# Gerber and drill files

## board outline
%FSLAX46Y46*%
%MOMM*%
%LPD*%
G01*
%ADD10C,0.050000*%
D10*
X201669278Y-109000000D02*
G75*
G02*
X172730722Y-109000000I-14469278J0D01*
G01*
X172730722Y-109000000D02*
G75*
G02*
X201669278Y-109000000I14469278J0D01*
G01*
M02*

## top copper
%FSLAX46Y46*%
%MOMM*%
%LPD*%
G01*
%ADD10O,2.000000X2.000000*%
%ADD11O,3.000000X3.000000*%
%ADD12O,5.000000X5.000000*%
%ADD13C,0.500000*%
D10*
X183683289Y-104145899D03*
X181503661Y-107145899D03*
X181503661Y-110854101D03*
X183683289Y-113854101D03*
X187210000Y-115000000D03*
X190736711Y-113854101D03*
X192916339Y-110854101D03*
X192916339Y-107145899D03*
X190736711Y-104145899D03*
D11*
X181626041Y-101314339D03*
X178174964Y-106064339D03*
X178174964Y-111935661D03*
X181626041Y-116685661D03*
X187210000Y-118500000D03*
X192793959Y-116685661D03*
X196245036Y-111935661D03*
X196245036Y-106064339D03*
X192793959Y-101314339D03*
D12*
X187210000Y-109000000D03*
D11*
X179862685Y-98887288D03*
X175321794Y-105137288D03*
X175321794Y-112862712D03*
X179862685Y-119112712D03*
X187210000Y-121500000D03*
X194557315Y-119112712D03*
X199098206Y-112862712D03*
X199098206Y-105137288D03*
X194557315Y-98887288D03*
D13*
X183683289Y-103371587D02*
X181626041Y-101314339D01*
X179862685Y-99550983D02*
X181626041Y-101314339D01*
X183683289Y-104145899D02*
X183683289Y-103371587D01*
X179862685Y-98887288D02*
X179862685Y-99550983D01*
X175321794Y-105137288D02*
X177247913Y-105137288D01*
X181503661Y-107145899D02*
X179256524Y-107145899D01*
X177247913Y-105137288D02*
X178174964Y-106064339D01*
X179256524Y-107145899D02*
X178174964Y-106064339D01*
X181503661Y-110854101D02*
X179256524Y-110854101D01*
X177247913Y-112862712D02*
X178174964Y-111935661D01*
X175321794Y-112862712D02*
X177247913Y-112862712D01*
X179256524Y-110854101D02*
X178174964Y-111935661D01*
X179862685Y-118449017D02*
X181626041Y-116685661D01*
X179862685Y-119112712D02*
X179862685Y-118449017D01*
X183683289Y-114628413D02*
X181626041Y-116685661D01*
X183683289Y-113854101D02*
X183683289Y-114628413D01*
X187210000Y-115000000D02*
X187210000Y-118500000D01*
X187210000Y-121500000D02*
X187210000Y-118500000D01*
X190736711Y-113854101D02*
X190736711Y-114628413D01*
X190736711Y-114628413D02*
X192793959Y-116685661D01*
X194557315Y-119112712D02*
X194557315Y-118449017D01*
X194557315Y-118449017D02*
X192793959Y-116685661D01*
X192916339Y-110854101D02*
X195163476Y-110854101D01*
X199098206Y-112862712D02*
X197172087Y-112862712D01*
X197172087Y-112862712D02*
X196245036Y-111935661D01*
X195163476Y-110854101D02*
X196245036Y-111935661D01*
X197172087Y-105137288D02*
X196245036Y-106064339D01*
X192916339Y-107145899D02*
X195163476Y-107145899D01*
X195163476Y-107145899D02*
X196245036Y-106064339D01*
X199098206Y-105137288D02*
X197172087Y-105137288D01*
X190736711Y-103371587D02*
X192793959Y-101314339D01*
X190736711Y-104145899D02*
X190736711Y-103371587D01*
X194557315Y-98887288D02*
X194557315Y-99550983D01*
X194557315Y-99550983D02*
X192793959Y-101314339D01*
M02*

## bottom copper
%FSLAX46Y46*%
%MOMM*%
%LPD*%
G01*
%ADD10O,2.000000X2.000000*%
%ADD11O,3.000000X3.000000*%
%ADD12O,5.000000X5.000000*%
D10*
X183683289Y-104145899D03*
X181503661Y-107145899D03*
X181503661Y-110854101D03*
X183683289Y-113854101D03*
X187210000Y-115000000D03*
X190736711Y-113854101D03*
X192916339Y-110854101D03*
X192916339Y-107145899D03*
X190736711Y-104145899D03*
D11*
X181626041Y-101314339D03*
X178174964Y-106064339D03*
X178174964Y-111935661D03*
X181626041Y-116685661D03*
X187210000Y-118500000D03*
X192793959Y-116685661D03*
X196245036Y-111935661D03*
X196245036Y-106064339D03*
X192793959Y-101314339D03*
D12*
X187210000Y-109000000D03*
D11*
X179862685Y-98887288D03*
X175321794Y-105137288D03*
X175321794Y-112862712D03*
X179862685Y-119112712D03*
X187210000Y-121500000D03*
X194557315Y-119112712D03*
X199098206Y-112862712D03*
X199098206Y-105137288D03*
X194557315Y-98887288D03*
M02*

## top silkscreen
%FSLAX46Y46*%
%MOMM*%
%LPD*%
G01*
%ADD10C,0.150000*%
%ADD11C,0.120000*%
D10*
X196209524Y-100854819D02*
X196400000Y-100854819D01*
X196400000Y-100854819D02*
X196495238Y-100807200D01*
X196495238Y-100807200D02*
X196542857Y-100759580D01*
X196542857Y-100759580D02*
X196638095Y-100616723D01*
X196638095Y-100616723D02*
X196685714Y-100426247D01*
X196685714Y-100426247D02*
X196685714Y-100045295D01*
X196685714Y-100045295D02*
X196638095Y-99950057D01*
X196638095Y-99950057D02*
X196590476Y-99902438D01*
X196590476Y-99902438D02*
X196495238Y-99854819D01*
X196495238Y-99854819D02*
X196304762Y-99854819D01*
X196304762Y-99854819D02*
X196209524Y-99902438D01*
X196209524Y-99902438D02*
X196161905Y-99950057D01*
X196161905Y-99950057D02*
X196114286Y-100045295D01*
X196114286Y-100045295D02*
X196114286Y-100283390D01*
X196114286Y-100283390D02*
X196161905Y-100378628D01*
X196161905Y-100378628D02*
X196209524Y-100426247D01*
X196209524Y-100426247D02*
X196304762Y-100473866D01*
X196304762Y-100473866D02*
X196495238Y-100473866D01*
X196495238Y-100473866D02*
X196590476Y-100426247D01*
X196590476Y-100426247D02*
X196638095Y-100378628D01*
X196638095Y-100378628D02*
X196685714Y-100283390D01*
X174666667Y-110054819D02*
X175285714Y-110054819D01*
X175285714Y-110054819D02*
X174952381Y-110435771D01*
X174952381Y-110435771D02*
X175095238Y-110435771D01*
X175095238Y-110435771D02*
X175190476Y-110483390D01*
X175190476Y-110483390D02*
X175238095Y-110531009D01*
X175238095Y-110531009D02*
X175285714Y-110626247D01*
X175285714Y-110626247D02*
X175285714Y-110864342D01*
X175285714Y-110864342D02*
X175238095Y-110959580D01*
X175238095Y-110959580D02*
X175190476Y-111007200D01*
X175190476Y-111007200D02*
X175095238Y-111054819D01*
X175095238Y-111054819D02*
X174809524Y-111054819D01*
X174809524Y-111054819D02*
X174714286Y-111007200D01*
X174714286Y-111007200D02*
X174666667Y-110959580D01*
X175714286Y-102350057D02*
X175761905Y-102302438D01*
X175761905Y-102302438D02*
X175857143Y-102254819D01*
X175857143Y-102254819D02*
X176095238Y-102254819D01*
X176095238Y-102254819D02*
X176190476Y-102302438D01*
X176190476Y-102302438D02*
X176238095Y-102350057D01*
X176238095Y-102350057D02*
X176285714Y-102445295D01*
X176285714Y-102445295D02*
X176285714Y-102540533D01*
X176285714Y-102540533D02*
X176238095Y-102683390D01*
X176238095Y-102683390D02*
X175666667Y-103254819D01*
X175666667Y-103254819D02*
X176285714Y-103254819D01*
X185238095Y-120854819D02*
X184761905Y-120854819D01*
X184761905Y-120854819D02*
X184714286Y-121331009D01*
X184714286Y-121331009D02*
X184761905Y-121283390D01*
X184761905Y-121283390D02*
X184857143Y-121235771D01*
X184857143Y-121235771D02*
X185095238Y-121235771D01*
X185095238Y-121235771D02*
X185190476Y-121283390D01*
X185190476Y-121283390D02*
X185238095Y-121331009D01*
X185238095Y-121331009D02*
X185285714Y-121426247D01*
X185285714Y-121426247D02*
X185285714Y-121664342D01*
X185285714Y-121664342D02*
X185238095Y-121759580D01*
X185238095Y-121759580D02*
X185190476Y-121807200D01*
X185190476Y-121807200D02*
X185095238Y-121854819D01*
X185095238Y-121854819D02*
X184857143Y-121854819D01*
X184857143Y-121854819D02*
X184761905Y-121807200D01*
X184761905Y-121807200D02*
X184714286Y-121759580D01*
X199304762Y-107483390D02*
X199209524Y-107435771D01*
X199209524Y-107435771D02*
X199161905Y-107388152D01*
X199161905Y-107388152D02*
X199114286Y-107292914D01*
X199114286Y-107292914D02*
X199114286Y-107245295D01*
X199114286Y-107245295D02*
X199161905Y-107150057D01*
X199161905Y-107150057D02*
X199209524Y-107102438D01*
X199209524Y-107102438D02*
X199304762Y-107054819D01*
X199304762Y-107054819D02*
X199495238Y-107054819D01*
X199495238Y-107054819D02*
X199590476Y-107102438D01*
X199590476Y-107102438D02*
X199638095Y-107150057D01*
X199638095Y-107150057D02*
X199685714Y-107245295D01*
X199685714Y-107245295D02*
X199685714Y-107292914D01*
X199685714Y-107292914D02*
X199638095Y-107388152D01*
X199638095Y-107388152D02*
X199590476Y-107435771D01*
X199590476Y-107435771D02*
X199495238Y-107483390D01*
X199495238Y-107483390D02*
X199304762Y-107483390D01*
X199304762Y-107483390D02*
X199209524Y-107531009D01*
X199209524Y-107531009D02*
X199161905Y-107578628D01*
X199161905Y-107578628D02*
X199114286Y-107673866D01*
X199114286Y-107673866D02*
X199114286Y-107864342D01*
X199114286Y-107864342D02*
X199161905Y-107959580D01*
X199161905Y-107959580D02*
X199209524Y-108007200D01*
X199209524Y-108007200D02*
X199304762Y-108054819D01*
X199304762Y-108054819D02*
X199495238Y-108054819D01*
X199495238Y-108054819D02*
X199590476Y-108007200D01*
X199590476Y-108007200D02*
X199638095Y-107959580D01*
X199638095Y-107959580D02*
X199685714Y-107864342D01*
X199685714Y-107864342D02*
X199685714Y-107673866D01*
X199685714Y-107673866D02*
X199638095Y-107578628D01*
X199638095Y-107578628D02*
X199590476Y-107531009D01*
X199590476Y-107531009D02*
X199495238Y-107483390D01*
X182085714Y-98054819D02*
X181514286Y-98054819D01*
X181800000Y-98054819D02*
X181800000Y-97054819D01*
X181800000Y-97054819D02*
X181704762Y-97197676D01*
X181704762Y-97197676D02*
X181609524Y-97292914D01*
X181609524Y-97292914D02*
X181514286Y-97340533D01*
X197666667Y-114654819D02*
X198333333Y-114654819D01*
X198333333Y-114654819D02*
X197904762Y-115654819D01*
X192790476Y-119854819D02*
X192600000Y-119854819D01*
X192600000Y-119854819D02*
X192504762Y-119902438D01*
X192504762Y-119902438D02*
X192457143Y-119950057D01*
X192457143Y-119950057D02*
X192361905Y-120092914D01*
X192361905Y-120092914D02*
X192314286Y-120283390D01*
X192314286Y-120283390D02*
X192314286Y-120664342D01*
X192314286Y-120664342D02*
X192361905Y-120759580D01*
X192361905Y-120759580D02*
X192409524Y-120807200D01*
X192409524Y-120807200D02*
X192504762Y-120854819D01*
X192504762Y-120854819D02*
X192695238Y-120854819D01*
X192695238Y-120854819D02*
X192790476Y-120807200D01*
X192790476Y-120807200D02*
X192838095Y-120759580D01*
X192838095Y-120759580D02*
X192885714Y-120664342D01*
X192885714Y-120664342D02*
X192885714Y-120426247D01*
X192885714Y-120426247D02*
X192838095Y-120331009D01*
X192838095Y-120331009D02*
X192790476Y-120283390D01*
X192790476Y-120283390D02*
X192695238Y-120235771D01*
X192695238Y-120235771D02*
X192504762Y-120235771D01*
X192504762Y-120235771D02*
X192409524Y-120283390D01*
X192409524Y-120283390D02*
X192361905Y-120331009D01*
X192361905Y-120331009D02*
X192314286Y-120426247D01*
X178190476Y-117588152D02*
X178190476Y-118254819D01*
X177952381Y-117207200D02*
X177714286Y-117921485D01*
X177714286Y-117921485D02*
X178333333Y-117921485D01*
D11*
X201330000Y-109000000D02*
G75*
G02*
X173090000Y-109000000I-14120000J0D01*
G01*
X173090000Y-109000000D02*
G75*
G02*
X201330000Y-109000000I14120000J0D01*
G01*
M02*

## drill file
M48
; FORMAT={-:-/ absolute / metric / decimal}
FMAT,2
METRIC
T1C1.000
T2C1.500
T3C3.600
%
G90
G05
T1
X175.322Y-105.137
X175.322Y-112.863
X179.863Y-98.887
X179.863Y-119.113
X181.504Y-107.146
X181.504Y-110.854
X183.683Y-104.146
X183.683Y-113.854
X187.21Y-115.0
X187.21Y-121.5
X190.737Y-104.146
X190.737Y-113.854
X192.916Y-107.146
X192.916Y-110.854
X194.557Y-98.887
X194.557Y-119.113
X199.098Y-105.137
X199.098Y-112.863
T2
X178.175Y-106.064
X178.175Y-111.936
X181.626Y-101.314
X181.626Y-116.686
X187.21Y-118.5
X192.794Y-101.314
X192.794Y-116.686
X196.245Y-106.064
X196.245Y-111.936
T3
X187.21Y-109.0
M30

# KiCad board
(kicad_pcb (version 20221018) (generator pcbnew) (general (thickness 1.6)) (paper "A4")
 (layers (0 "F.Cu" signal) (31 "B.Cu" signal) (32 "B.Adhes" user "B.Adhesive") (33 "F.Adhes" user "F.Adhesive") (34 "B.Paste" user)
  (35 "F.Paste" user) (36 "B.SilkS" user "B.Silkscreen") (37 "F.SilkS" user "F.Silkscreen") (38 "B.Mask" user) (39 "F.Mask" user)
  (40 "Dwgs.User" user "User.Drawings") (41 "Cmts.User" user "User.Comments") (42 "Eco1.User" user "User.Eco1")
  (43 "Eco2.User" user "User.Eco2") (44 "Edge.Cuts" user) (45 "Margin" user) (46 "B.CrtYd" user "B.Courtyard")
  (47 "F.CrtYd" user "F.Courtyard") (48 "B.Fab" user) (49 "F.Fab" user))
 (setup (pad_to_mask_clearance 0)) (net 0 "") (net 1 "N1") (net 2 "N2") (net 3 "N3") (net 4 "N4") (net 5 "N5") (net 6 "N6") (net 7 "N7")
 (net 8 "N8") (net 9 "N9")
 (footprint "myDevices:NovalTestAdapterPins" (layer "F.Cu") (at 187.21 109)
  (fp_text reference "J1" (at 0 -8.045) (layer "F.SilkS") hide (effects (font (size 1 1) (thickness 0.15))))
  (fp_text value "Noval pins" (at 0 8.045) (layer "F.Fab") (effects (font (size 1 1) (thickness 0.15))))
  (pad "1" thru_hole oval (at -3.526711 -4.854101) (size 2 2) (drill 1) (layers "*.Cu" "*.Mask") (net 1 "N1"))
  (pad "2" thru_hole oval (at -5.706339 -1.854101) (size 2 2) (drill 1) (layers "*.Cu" "*.Mask") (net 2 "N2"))
  (pad "3" thru_hole oval (at -5.706339 1.854101) (size 2 2) (drill 1) (layers "*.Cu" "*.Mask") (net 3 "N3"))
  (pad "4" thru_hole oval (at -3.526711 4.854101) (size 2 2) (drill 1) (layers "*.Cu" "*.Mask") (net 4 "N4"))
  (pad "5" thru_hole oval (at 0 6) (size 2 2) (drill 1) (layers "*.Cu" "*.Mask") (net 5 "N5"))
  (pad "6" thru_hole oval (at 3.526711 4.854101) (size 2 2) (drill 1) (layers "*.Cu" "*.Mask") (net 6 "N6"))
  (pad "7" thru_hole oval (at 5.706339 1.854101) (size 2 2) (drill 1) (layers "*.Cu" "*.Mask") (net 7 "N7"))
  (pad "8" thru_hole oval (at 5.706339 -1.854101) (size 2 2) (drill 1) (layers "*.Cu" "*.Mask") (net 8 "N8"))
  (pad "9" thru_hole oval (at 3.526711 -4.854101) (size 2 2) (drill 1) (layers "*.Cu" "*.Mask") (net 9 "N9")))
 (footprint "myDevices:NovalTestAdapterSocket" (layer "F.Cu") (at 187.21 109)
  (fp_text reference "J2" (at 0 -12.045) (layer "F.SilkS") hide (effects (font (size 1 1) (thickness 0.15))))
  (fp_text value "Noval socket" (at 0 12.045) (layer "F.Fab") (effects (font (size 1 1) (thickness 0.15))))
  (pad "1" thru_hole oval (at -5.583959 -7.685661) (size 3 3) (drill 1.5) (layers "*.Cu" "*.Mask") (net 1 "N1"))
  (pad "2" thru_hole oval (at -9.035036 -2.935661) (size 3 3) (drill 1.5) (layers "*.Cu" "*.Mask") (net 2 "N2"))
  (pad "3" thru_hole oval (at -9.035036 2.935661) (size 3 3) (drill 1.5) (layers "*.Cu" "*.Mask") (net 3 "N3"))
  (pad "4" thru_hole oval (at -5.583959 7.685661) (size 3 3) (drill 1.5) (layers "*.Cu" "*.Mask") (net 4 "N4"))
  (pad "5" thru_hole oval (at 0 9.5) (size 3 3) (drill 1.5) (layers "*.Cu" "*.Mask") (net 5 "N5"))
  (pad "6" thru_hole oval (at 5.583959 7.685661) (size 3 3) (drill 1.5) (layers "*.Cu" "*.Mask") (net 6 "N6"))
  (pad "7" thru_hole oval (at 9.035036 2.935661) (size 3 3) (drill 1.5) (layers "*.Cu" "*.Mask") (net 7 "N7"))
  (pad "8" thru_hole oval (at 9.035036 -2.935661) (size 3 3) (drill 1.5) (layers "*.Cu" "*.Mask") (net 8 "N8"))
  (pad "9" thru_hole oval (at 5.583959 -7.685661) (size 3 3) (drill 1.5) (layers "*.Cu" "*.Mask") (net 9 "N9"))
  (pad "10" thru_hole oval (at 0 0) (size 5 5) (drill 3.6) (layers "*.Cu" "*.Mask")))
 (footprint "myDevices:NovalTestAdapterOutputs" (layer "F.Cu") (at 187.21 109)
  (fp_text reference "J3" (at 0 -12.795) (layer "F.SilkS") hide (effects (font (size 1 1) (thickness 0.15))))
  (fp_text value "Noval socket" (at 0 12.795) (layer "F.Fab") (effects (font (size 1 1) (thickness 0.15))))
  (fp_circle (center 0 0) (end 0 14.12) (stroke (width 0.12) (type solid)) (fill none) (layer "F.SilkS"))
  (pad "1" thru_hole oval (at -7.347315 -10.112712) (size 3 3) (drill 1) (layers "*.Cu" "*.Mask") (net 1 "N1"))
  (pad "2" thru_hole oval (at -11.888206 -3.862712) (size 3 3) (drill 1) (layers "*.Cu" "*.Mask") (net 2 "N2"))
  (pad "3" thru_hole oval (at -11.888206 3.862712) (size 3 3) (drill 1) (layers "*.Cu" "*.Mask") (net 3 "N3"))
  (pad "4" thru_hole oval (at -7.347315 10.112712) (size 3 3) (drill 1) (layers "*.Cu" "*.Mask") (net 4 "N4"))
  (pad "5" thru_hole oval (at 0 12.5) (size 3 3) (drill 1) (layers "*.Cu" "*.Mask") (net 5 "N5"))
  (pad "6" thru_hole oval (at 7.347315 10.112712) (size 3 3) (drill 1) (layers "*.Cu" "*.Mask") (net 6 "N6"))
  (pad "7" thru_hole oval (at 11.888206 3.862712) (size 3 3) (drill 1) (layers "*.Cu" "*.Mask") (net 7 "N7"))
  (pad "8" thru_hole oval (at 11.888206 -3.862712) (size 3 3) (drill 1) (layers "*.Cu" "*.Mask") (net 8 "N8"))
  (pad "9" thru_hole oval (at 7.347315 -10.112712) (size 3 3) (drill 1) (layers "*.Cu" "*.Mask") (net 9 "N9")))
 (gr_circle (center 187.2 109) (end 198.2 118.4) (stroke (width 0.05) (type solid)) (fill none) (layer "Edge.Cuts"))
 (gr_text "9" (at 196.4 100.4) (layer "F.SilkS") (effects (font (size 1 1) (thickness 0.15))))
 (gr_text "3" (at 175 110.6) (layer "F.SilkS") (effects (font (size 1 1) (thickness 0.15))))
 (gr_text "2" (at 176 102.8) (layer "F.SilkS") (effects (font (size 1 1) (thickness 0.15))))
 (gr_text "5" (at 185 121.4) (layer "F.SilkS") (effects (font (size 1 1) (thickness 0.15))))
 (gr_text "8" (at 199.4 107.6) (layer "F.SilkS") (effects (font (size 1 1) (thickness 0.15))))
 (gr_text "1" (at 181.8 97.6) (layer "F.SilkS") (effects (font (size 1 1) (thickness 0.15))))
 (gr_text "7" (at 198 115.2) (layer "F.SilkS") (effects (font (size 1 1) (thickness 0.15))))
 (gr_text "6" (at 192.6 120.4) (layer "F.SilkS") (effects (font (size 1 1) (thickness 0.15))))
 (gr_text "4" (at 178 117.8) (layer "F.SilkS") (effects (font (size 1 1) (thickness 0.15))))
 (segment (start 183.683289 103.371587) (end 181.626041 101.314339) (width 0.5) (layer "F.Cu") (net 1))
 (segment (start 179.862685 99.550983) (end 181.626041 101.314339) (width 0.5) (layer "F.Cu") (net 1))
 (segment (start 183.683289 104.145899) (end 183.683289 103.371587) (width 0.5) (layer "F.Cu") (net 1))
 (segment (start 179.862685 98.887288) (end 179.862685 99.550983) (width 0.5) (layer "F.Cu") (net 1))
 (segment (start 175.321794 105.137288) (end 177.247913 105.137288) (width 0.5) (layer "F.Cu") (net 2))
 (segment (start 181.503661 107.145899) (end 179.256524 107.145899) (width 0.5) (layer "F.Cu") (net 2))
 (segment (start 177.247913 105.137288) (end 178.174964 106.064339) (width 0.5) (layer "F.Cu") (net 2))
 (segment (start 179.256524 107.145899) (end 178.174964 106.064339) (width 0.5) (layer "F.Cu") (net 2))
 (segment (start 181.503661 110.854101) (end 179.256524 110.854101) (width 0.5) (layer "F.Cu") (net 3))
 (segment (start 177.247913 112.862712) (end 178.174964 111.935661) (width 0.5) (layer "F.Cu") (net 3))
 (segment (start 175.321794 112.862712) (end 177.247913 112.862712) (width 0.5) (layer "F.Cu") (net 3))
 (segment (start 179.256524 110.854101) (end 178.174964 111.935661) (width 0.5) (layer "F.Cu") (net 3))
 (segment (start 179.862685 118.449017) (end 181.626041 116.685661) (width 0.5) (layer "F.Cu") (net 4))
 (segment (start 179.862685 119.112712) (end 179.862685 118.449017) (width 0.5) (layer "F.Cu") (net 4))
 (segment (start 183.683289 114.628413) (end 181.626041 116.685661) (width 0.5) (layer "F.Cu") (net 4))
 (segment (start 183.683289 113.854101) (end 183.683289 114.628413) (width 0.5) (layer "F.Cu") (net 4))
 (segment (start 187.21 115) (end 187.21 118.5) (width 0.5) (layer "F.Cu") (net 5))
 (segment (start 187.21 121.5) (end 187.21 118.5) (width 0.5) (layer "F.Cu") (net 5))
 (segment (start 190.736711 113.854101) (end 190.736711 114.628413) (width 0.5) (layer "F.Cu") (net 6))
 (segment (start 190.736711 114.628413) (end 192.793959 116.685661) (width 0.5) (layer "F.Cu") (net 6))
 (segment (start 194.557315 119.112712) (end 194.557315 118.449017) (width 0.5) (layer "F.Cu") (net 6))
 (segment (start 194.557315 118.449017) (end 192.793959 116.685661) (width 0.5) (layer "F.Cu") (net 6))
 (segment (start 192.916339 110.854101) (end 195.163476 110.854101) (width 0.5) (layer "F.Cu") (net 7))
 (segment (start 199.098206 112.862712) (end 197.172087 112.862712) (width 0.5) (layer "F.Cu") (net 7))
 (segment (start 197.172087 112.862712) (end 196.245036 111.935661) (width 0.5) (layer "F.Cu") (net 7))
 (segment (start 195.163476 110.854101) (end 196.245036 111.935661) (width 0.5) (layer "F.Cu") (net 7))
 (segment (start 197.172087 105.137288) (end 196.245036 106.064339) (width 0.5) (layer "F.Cu") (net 8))
 (segment (start 192.916339 107.145899) (end 195.163476 107.145899) (width 0.5) (layer "F.Cu") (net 8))
 (segment (start 195.163476 107.145899) (end 196.245036 106.064339) (width 0.5) (layer "F.Cu") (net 8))
 (segment (start 199.098206 105.137288) (end 197.172087 105.137288) (width 0.5) (layer "F.Cu") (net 8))
 (segment (start 190.736711 103.371587) (end 192.793959 101.314339) (width 0.5) (layer "F.Cu") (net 9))
 (segment (start 190.736711 104.145899) (end 190.736711 103.371587) (width 0.5) (layer "F.Cu") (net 9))
 (segment (start 194.557315 98.887288) (end 194.557315 99.550983) (width 0.5) (layer "F.Cu") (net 9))
 (segment (start 194.557315 99.550983) (end 192.793959 101.314339) (width 0.5) (layer "F.Cu") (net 9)))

